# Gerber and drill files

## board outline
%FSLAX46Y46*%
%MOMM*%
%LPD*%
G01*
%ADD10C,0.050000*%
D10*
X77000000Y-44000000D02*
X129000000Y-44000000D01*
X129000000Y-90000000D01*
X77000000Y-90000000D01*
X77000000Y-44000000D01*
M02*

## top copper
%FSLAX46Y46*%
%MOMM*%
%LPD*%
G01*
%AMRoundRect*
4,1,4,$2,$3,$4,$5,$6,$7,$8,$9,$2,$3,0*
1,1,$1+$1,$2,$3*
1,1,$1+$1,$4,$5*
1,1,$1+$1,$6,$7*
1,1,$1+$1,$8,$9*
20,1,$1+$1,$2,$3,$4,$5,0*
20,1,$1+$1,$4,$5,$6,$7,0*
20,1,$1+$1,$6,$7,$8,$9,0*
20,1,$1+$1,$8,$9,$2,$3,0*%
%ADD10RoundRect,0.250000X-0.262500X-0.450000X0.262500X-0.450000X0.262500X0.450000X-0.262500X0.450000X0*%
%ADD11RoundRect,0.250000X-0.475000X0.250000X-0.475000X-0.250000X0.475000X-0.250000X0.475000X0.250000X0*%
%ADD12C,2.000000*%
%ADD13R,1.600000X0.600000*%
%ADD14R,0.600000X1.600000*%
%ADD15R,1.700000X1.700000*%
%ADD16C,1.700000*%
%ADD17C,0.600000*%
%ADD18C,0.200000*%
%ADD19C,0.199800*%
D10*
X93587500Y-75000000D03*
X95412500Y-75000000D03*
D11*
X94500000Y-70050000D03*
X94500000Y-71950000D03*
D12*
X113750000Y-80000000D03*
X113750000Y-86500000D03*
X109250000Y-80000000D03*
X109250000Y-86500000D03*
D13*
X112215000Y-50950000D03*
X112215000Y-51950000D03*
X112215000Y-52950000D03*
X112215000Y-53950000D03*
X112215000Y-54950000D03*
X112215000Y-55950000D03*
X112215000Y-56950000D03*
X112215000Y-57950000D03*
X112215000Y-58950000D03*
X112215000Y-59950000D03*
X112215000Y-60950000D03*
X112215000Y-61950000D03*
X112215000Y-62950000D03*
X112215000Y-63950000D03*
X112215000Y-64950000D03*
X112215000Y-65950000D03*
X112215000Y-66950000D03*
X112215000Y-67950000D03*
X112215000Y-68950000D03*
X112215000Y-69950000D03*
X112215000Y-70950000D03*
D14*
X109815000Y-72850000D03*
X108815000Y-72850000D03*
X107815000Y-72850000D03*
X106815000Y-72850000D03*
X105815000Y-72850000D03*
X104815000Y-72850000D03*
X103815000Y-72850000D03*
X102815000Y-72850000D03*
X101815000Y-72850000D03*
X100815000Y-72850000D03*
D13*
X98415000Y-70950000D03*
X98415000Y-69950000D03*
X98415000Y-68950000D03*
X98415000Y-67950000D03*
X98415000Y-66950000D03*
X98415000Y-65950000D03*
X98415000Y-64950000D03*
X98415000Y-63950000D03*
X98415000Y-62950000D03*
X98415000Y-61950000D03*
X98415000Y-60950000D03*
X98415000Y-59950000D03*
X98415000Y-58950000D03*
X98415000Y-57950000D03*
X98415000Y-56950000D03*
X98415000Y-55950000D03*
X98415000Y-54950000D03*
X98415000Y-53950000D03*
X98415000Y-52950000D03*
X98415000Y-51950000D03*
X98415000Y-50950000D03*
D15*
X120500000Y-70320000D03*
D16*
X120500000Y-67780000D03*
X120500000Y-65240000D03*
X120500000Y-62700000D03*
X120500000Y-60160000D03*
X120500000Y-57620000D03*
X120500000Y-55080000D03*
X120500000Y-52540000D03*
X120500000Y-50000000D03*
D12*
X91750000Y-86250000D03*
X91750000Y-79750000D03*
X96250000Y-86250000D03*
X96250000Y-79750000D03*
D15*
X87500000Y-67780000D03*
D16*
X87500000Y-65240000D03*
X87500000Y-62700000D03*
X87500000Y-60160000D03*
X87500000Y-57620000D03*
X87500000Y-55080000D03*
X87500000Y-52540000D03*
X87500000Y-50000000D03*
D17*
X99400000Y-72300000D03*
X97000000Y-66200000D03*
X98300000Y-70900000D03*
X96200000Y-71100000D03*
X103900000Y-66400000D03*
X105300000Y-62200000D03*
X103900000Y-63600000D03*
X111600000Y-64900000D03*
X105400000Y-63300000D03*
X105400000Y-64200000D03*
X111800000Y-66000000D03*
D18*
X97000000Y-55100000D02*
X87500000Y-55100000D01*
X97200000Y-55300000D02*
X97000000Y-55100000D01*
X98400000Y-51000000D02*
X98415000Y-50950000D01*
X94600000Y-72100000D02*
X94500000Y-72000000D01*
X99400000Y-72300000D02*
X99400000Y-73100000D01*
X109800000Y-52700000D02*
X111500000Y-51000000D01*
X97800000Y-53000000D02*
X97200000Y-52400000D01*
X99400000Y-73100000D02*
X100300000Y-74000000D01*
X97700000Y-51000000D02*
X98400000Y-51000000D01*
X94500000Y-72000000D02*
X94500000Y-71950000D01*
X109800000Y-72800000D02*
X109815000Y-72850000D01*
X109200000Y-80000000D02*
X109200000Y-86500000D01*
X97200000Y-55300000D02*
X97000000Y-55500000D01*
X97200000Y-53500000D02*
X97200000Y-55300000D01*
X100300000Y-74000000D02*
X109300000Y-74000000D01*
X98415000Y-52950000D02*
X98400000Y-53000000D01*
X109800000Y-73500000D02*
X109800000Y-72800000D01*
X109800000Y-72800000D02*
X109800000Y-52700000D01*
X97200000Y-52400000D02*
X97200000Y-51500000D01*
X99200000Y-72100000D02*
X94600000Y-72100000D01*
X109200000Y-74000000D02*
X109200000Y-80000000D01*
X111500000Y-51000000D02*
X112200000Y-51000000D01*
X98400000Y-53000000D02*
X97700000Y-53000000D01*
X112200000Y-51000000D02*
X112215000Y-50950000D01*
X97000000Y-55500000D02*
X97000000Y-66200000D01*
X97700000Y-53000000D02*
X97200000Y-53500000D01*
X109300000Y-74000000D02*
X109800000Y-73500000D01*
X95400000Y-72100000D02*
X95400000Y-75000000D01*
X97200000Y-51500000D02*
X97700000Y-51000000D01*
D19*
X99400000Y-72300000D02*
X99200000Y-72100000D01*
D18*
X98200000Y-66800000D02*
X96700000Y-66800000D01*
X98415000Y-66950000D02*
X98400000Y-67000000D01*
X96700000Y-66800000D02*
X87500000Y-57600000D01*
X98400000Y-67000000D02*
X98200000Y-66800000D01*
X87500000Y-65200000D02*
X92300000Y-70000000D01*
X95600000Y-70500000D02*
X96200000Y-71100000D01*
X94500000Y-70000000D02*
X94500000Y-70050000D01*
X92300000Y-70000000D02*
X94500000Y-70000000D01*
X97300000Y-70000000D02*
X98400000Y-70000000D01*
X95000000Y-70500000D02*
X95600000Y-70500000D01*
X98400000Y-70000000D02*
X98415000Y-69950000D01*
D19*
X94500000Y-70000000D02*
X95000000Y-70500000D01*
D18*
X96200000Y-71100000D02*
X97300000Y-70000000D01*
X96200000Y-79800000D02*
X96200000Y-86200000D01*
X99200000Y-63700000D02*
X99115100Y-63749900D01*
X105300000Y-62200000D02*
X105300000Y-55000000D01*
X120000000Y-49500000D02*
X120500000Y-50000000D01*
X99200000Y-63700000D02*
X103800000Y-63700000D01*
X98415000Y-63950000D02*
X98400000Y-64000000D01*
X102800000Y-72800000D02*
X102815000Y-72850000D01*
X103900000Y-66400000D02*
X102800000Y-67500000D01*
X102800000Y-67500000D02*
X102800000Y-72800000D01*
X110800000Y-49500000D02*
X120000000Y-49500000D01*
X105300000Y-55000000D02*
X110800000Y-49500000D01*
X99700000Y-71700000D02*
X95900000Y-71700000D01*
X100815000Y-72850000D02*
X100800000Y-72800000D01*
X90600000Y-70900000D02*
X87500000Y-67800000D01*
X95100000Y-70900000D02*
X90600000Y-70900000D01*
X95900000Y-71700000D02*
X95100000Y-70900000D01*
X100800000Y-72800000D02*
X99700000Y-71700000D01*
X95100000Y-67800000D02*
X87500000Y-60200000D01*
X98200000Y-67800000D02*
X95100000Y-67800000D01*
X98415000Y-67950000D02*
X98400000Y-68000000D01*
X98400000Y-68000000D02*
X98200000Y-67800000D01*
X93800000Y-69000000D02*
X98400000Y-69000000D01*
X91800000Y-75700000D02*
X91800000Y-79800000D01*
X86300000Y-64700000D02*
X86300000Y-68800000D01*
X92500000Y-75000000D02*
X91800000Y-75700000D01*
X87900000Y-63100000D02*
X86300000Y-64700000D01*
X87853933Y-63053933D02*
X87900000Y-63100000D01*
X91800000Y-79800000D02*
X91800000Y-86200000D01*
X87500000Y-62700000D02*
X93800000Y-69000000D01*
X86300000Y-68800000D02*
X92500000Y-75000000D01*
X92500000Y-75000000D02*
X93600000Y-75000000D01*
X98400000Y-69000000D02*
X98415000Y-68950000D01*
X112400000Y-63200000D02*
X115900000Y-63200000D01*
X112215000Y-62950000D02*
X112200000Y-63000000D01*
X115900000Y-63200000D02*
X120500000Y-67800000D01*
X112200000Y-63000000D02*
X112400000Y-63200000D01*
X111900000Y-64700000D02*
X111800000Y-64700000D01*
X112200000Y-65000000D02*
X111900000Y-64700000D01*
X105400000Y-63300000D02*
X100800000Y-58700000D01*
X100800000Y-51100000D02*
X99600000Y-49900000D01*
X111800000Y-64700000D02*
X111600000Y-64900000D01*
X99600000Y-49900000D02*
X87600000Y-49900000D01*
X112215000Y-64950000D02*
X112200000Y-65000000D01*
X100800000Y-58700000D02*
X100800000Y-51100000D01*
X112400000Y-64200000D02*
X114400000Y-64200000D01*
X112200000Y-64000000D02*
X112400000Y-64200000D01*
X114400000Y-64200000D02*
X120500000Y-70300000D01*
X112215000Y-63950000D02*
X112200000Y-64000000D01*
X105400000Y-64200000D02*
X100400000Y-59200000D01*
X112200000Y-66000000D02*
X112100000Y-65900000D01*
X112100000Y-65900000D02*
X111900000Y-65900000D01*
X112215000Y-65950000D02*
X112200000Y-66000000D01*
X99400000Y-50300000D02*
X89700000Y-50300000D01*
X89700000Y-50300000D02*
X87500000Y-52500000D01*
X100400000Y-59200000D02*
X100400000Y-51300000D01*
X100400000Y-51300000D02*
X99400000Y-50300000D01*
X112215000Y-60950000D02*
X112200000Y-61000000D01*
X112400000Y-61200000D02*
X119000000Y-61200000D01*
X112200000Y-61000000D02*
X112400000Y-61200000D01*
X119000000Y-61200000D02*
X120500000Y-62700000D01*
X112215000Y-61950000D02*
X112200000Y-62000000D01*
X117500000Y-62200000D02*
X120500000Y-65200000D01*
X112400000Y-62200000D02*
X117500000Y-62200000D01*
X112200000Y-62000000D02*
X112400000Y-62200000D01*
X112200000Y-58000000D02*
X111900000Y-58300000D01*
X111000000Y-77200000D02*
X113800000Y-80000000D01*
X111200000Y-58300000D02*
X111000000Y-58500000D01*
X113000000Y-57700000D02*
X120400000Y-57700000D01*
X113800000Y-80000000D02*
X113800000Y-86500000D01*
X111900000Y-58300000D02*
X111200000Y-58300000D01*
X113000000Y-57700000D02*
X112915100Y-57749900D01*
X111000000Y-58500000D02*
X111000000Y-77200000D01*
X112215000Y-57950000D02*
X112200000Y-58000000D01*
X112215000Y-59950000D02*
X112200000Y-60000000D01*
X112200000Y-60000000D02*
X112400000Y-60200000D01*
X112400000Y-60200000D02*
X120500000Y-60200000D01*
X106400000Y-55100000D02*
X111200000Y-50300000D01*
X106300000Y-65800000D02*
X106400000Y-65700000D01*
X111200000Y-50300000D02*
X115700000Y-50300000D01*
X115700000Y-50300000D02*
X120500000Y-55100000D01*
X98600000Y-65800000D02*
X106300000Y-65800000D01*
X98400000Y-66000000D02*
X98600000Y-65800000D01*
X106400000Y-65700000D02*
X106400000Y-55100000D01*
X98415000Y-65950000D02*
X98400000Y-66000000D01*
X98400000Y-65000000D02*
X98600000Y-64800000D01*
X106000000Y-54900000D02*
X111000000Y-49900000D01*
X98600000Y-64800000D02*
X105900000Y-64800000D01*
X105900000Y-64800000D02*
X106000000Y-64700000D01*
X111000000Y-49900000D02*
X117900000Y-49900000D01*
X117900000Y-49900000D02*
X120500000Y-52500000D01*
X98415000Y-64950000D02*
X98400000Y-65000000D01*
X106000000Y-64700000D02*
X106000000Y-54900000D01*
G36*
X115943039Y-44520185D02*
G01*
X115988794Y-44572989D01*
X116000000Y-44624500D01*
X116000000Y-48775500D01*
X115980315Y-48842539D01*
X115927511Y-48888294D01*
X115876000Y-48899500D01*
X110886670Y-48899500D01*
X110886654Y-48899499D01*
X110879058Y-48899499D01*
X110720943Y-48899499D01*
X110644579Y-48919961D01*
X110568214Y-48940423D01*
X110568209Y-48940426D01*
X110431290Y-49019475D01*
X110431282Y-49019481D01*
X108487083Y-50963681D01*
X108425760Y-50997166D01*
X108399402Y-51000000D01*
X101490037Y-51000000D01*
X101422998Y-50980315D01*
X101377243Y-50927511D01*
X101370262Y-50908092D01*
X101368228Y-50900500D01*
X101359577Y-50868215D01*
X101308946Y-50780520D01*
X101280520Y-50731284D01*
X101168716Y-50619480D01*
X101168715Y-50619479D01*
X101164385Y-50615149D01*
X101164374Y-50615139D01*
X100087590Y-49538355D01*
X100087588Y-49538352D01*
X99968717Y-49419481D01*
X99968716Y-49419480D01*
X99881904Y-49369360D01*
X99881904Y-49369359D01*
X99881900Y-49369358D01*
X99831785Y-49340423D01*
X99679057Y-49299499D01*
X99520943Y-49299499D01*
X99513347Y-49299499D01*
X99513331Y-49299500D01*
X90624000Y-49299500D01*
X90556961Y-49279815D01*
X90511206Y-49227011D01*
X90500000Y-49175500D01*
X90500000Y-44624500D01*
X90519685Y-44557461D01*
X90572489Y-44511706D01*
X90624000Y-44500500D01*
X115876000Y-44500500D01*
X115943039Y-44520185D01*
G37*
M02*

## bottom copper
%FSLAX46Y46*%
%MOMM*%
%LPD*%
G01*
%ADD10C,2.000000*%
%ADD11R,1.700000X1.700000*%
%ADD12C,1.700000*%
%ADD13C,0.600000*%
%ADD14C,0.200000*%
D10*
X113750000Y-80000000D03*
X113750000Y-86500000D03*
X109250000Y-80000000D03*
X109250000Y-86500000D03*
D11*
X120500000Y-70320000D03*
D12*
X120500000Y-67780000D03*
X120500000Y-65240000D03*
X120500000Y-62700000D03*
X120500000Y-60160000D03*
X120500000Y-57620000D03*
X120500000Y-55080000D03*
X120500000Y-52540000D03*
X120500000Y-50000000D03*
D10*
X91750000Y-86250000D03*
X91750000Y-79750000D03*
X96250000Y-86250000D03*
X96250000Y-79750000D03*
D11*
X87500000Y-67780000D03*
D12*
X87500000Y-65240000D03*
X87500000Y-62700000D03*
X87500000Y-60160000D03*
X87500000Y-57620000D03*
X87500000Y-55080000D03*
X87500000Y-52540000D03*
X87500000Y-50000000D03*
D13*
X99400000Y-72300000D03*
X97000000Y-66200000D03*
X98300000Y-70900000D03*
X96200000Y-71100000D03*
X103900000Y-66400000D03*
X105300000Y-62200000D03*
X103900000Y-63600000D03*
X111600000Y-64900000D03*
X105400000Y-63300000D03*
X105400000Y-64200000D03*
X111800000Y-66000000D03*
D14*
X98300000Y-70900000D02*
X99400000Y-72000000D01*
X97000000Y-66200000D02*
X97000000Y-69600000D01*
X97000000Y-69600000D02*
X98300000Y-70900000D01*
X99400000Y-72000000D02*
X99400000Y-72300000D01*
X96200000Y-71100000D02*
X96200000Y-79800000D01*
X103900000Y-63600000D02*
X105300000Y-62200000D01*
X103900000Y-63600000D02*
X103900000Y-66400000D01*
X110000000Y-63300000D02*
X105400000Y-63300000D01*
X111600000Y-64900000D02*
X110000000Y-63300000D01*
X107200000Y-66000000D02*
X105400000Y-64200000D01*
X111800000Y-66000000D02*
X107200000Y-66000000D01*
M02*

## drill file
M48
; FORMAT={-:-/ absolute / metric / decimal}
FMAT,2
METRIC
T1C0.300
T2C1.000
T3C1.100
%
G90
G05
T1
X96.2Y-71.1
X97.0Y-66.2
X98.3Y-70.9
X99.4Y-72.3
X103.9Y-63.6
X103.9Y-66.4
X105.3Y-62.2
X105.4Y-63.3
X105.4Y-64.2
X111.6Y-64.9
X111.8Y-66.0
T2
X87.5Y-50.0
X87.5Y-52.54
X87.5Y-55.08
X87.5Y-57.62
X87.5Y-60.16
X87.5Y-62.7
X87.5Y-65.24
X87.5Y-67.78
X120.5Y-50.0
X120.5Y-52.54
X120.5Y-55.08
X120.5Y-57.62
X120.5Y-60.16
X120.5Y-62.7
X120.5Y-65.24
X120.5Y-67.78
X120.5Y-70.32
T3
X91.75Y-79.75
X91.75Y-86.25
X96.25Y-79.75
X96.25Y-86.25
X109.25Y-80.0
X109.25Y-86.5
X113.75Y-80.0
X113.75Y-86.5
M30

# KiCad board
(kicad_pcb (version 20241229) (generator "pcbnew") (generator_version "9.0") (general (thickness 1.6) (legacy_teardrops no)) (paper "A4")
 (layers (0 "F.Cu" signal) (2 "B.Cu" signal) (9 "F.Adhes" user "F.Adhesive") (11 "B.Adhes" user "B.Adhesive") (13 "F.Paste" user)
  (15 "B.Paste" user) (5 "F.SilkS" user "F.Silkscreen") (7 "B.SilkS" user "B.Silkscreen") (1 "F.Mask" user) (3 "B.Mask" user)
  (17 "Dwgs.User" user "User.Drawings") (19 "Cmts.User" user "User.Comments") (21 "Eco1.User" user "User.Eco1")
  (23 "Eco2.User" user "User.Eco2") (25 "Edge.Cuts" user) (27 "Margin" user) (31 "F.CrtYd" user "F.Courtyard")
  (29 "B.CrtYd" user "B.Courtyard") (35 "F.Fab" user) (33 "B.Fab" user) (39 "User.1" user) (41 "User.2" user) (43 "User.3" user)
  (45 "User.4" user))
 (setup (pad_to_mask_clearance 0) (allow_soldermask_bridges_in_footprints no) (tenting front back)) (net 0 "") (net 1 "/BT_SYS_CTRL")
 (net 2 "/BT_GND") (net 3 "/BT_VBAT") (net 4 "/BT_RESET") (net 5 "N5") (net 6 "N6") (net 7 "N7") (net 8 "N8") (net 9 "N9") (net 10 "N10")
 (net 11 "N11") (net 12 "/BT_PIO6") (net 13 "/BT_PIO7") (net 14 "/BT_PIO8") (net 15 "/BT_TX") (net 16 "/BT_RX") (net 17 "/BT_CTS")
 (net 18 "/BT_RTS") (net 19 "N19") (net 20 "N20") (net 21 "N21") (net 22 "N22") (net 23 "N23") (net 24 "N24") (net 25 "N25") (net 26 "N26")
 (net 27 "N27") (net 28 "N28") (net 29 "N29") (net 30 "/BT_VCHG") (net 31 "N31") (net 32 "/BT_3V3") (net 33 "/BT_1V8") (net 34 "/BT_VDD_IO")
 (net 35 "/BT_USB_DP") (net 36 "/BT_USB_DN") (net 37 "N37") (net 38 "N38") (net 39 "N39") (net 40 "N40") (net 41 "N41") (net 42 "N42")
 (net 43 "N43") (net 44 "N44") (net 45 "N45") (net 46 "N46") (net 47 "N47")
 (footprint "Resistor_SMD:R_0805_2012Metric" (layer "F.Cu") (at 94.5 75)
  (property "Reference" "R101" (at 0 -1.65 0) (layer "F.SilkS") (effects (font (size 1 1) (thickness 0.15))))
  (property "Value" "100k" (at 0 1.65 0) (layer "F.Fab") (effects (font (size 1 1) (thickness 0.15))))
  (pad "1" smd roundrect (at -0.9125 0) (size 1.025 1.4) (layers "F.Cu" "F.Mask" "F.Paste") (roundrect_rratio 0.243902)
   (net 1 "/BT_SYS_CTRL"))
  (pad "2" smd roundrect (at 0.9125 0) (size 1.025 1.4) (layers "F.Cu" "F.Mask" "F.Paste") (roundrect_rratio 0.243902) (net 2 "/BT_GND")))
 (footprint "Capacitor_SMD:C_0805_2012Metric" (layer "F.Cu") (at 94.5 71 -90)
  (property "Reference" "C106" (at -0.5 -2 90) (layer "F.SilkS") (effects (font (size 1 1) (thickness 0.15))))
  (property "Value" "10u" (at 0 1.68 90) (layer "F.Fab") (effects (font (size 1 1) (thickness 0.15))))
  (pad "1" smd roundrect (at -0.95 0 270) (size 1 1.45) (layers "F.Cu" "F.Mask" "F.Paste") (roundrect_rratio 0.25) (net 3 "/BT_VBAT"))
  (pad "2" smd roundrect (at 0.95 0 270) (size 1 1.45) (layers "F.Cu" "F.Mask" "F.Paste") (roundrect_rratio 0.25) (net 2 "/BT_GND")))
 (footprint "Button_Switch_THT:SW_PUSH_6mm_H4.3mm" (layer "F.Cu") (at 113.75 80 -90)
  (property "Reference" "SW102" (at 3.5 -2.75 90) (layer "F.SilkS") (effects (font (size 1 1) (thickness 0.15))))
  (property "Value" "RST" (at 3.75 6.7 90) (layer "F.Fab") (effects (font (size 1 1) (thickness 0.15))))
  (pad "1" thru_hole circle (at 0 0) (size 2 2) (drill 1.1) (layers "*.Cu" "*.Mask") (remove_unused_layers no) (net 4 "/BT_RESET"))
  (pad "1" thru_hole circle (at 6.5 0) (size 2 2) (drill 1.1) (layers "*.Cu" "*.Mask") (remove_unused_layers no) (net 4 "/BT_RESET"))
  (pad "2" thru_hole circle (at 0 4.5) (size 2 2) (drill 1.1) (layers "*.Cu" "*.Mask") (remove_unused_layers no) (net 2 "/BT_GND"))
  (pad "2" thru_hole circle (at 6.5 4.5) (size 2 2) (drill 1.1) (layers "*.Cu" "*.Mask") (remove_unused_layers no) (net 2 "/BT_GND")))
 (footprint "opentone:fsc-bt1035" (layer "F.Cu") (at 105.315 59 180)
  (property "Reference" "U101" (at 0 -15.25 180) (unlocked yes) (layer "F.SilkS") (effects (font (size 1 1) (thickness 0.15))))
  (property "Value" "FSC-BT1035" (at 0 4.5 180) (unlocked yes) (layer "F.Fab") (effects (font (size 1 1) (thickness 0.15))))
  (pad "1" smd rect (at -6.9 8.05 180) (size 1.6 0.6) (layers "F.Cu" "F.Mask" "F.Paste") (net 2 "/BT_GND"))
  (pad "2" smd rect (at -6.9 7.05 180) (size 1.6 0.6) (layers "F.Cu" "F.Mask" "F.Paste") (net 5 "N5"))
  (pad "3" smd rect (at -6.9 6.05 180) (size 1.6 0.6) (layers "F.Cu" "F.Mask" "F.Paste") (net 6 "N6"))
  (pad "4" smd rect (at -6.9 5.05 180) (size 1.6 0.6) (layers "F.Cu" "F.Mask" "F.Paste") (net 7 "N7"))
  (pad "5" smd rect (at -6.9 4.05 180) (size 1.6 0.6) (layers "F.Cu" "F.Mask" "F.Paste") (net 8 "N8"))
  (pad "6" smd rect (at -6.9 3.05 180) (size 1.6 0.6) (layers "F.Cu" "F.Mask" "F.Paste") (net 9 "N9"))
  (pad "7" smd rect (at -6.9 2.05 180) (size 1.6 0.6) (layers "F.Cu" "F.Mask" "F.Paste") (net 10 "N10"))
  (pad "8" smd rect (at -6.9 1.05 180) (size 1.6 0.6) (layers "F.Cu" "F.Mask" "F.Paste") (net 4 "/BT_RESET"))
  (pad "9" smd rect (at -6.9 0.05 180) (size 1.6 0.6) (layers "F.Cu" "F.Mask" "F.Paste") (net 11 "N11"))
  (pad "10" smd rect (at -6.9 -0.95 180) (size 1.6 0.6) (layers "F.Cu" "F.Mask" "F.Paste") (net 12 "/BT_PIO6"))
  (pad "11" smd rect (at -6.9 -1.95 180) (size 1.6 0.6) (layers "F.Cu" "F.Mask" "F.Paste") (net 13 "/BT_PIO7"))
  (pad "12" smd rect (at -6.9 -2.95 180) (size 1.6 0.6) (layers "F.Cu" "F.Mask" "F.Paste") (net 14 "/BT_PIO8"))
  (pad "13" smd rect (at -6.9 -3.95 180) (size 1.6 0.6) (layers "F.Cu" "F.Mask" "F.Paste") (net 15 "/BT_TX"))
  (pad "14" smd rect (at -6.9 -4.95 180) (size 1.6 0.6) (layers "F.Cu" "F.Mask" "F.Paste") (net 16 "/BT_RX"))
  (pad "15" smd rect (at -6.9 -5.95 180) (size 1.6 0.6) (layers "F.Cu" "F.Mask" "F.Paste") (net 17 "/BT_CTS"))
  (pad "16" smd rect (at -6.9 -6.95 180) (size 1.6 0.6) (layers "F.Cu" "F.Mask" "F.Paste") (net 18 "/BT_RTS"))
  (pad "17" smd rect (at -6.9 -7.95 180) (size 1.6 0.6) (layers "F.Cu" "F.Mask" "F.Paste") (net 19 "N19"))
  (pad "18" smd rect (at -6.9 -8.95 180) (size 1.6 0.6) (layers "F.Cu" "F.Mask" "F.Paste") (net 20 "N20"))
  (pad "19" smd rect (at -6.9 -9.95 180) (size 1.6 0.6) (layers "F.Cu" "F.Mask" "F.Paste") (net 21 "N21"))
  (pad "20" smd rect (at -6.9 -10.95 180) (size 1.6 0.6) (layers "F.Cu" "F.Mask" "F.Paste") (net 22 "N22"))
  (pad "21" smd rect (at -6.9 -11.95 180) (size 1.6 0.6) (layers "F.Cu" "F.Mask" "F.Paste") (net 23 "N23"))
  (pad "22" smd rect (at -4.5 -13.85 180) (size 0.6 1.6) (layers "F.Cu" "F.Mask" "F.Paste") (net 2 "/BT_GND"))
  (pad "23" smd rect (at -3.5 -13.85 180) (size 0.6 1.6) (layers "F.Cu" "F.Mask" "F.Paste") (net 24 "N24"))
  (pad "24" smd rect (at -2.5 -13.85 180) (size 0.6 1.6) (layers "F.Cu" "F.Mask" "F.Paste") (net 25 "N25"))
  (pad "25" smd rect (at -1.5 -13.85 180) (size 0.6 1.6) (layers "F.Cu" "F.Mask" "F.Paste") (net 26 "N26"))
  (pad "26" smd rect (at -0.5 -13.85 180) (size 0.6 1.6) (layers "F.Cu" "F.Mask" "F.Paste") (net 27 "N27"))
  (pad "27" smd rect (at 0.5 -13.85 180) (size 0.6 1.6) (layers "F.Cu" "F.Mask" "F.Paste") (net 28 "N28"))
  (pad "28" smd rect (at 1.5 -13.85 180) (size 0.6 1.6) (layers "F.Cu" "F.Mask" "F.Paste") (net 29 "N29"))
  (pad "29" smd rect (at 2.5 -13.85 180) (size 0.6 1.6) (layers "F.Cu" "F.Mask" "F.Paste") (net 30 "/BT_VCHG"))
  (pad "30" smd rect (at 3.5 -13.85 180) (size 0.6 1.6) (layers "F.Cu" "F.Mask" "F.Paste") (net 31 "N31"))
  (pad "31" smd rect (at 4.5 -13.85 180) (size 0.6 1.6) (layers "F.Cu" "F.Mask" "F.Paste") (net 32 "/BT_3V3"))
  (pad "32" smd rect (at 6.9 -11.95 180) (size 1.6 0.6) (layers "F.Cu" "F.Mask" "F.Paste") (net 2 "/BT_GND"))
  (pad "33" smd rect (at 6.9 -10.95 180) (size 1.6 0.6) (layers "F.Cu" "F.Mask" "F.Paste") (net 3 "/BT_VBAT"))
  (pad "34" smd rect (at 6.9 -9.95 180) (size 1.6 0.6) (layers "F.Cu" "F.Mask" "F.Paste") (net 1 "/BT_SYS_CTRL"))
  (pad "35" smd rect (at 6.9 -8.95 180) (size 1.6 0.6) (layers "F.Cu" "F.Mask" "F.Paste") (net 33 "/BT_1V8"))
  (pad "36" smd rect (at 6.9 -7.95 180) (size 1.6 0.6) (layers "F.Cu" "F.Mask" "F.Paste") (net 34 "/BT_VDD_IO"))
  (pad "37" smd rect (at 6.9 -6.95 180) (size 1.6 0.6) (layers "F.Cu" "F.Mask" "F.Paste") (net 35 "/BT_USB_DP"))
  (pad "38" smd rect (at 6.9 -5.95 180) (size 1.6 0.6) (layers "F.Cu" "F.Mask" "F.Paste") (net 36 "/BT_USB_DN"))
  (pad "39" smd rect (at 6.9 -4.95 180) (size 1.6 0.6) (layers "F.Cu" "F.Mask" "F.Paste") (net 30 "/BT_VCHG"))
  (pad "40" smd rect (at 6.9 -3.95 180) (size 1.6 0.6) (layers "F.Cu" "F.Mask" "F.Paste") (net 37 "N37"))
  (pad "41" smd rect (at 6.9 -2.95 180) (size 1.6 0.6) (layers "F.Cu" "F.Mask" "F.Paste") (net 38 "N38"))
  (pad "42" smd rect (at 6.9 -1.95 180) (size 1.6 0.6) (layers "F.Cu" "F.Mask" "F.Paste") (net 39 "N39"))
  (pad "43" smd rect (at 6.9 -0.95 180) (size 1.6 0.6) (layers "F.Cu" "F.Mask" "F.Paste") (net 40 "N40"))
  (pad "44" smd rect (at 6.9 0.05 180) (size 1.6 0.6) (layers "F.Cu" "F.Mask" "F.Paste") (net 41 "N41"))
  (pad "45" smd rect (at 6.9 1.05 180) (size 1.6 0.6) (layers "F.Cu" "F.Mask" "F.Paste") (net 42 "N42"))
  (pad "46" smd rect (at 6.9 2.05 180) (size 1.6 0.6) (layers "F.Cu" "F.Mask" "F.Paste") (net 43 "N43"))
  (pad "47" smd rect (at 6.9 3.05 180) (size 1.6 0.6) (layers "F.Cu" "F.Mask" "F.Paste") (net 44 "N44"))
  (pad "48" smd rect (at 6.9 4.05 180) (size 1.6 0.6) (layers "F.Cu" "F.Mask" "F.Paste") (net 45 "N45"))
  (pad "49" smd rect (at 6.9 5.05 180) (size 1.6 0.6) (layers "F.Cu" "F.Mask" "F.Paste") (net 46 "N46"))
  (pad "50" smd rect (at 6.9 6.05 180) (size 1.6 0.6) (layers "F.Cu" "F.Mask" "F.Paste") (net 2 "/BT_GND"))
  (pad "51" smd rect (at 6.9 7.05 180) (size 1.6 0.6) (layers "F.Cu" "F.Mask" "F.Paste") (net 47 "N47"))
  (pad "52" smd rect (at 6.9 8.05 180) (size 1.6 0.6) (layers "F.Cu" "F.Mask" "F.Paste") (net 2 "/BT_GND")))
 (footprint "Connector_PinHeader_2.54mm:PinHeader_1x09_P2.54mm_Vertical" (layer "F.Cu") (at 120.5 70.32 180)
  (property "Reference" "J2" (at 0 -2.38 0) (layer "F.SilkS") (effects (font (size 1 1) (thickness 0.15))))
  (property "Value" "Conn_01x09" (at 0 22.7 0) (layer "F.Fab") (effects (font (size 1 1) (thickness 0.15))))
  (pad "1" thru_hole rect (at 0 0 180) (size 1.7 1.7) (drill 1) (layers "*.Cu" "*.Mask") (remove_unused_layers no) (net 16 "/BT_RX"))
  (pad "2" thru_hole circle (at 0 2.54 180) (size 1.7 1.7) (drill 1) (layers "*.Cu" "*.Mask") (remove_unused_layers no) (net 15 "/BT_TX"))
  (pad "3" thru_hole circle (at 0 5.08 180) (size 1.7 1.7) (drill 1) (layers "*.Cu" "*.Mask") (remove_unused_layers no) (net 14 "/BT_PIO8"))
  (pad "4" thru_hole circle (at 0 7.62 180) (size 1.7 1.7) (drill 1) (layers "*.Cu" "*.Mask") (remove_unused_layers no) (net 13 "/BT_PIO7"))
  (pad "5" thru_hole circle (at 0 10.16 180) (size 1.7 1.7) (drill 1) (layers "*.Cu" "*.Mask") (remove_unused_layers no) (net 12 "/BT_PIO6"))
  (pad "6" thru_hole circle (at 0 12.7 180) (size 1.7 1.7) (drill 1) (layers "*.Cu" "*.Mask") (remove_unused_layers no) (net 4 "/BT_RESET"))
  (pad "7" thru_hole circle (at 0 15.24 180) (size 1.7 1.7) (drill 1) (layers "*.Cu" "*.Mask") (remove_unused_layers no)
   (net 35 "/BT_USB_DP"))
  (pad "8" thru_hole circle (at 0 17.78 180) (size 1.7 1.7) (drill 1) (layers "*.Cu" "*.Mask") (remove_unused_layers no)
   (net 36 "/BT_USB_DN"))
  (pad "9" thru_hole circle (at 0 20.32 180) (size 1.7 1.7) (drill 1) (layers "*.Cu" "*.Mask") (remove_unused_layers no) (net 30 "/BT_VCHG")))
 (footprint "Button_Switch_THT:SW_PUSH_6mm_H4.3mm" (layer "F.Cu") (at 91.75 86.25 90)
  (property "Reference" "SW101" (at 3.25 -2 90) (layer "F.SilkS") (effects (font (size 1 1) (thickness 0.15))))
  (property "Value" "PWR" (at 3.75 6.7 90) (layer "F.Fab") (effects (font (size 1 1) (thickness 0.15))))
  (pad "1" thru_hole circle (at 0 0 180) (size 2 2) (drill 1.1) (layers "*.Cu" "*.Mask") (remove_unused_layers no) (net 1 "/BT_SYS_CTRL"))
  (pad "1" thru_hole circle (at 6.5 0 180) (size 2 2) (drill 1.1) (layers "*.Cu" "*.Mask") (remove_unused_layers no) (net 1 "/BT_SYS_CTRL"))
  (pad "2" thru_hole circle (at 0 4.5 180) (size 2 2) (drill 1.1) (layers "*.Cu" "*.Mask") (remove_unused_layers no) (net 3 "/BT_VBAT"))
  (pad "2" thru_hole circle (at 6.5 4.5 180) (size 2 2) (drill 1.1) (layers "*.Cu" "*.Mask") (remove_unused_layers no) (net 3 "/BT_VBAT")))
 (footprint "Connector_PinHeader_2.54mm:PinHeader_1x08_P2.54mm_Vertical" (layer "F.Cu") (at 87.5 67.78 180)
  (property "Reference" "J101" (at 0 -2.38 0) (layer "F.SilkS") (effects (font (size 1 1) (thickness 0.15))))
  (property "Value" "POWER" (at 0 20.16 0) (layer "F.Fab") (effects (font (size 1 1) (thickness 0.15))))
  (pad "1" thru_hole rect (at 0 0 180) (size 1.7 1.7) (drill 1) (layers "*.Cu" "*.Mask") (remove_unused_layers no) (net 32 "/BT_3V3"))
  (pad "2" thru_hole circle (at 0 2.54 180) (size 1.7 1.7) (drill 1) (layers "*.Cu" "*.Mask") (remove_unused_layers no) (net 3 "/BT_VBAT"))
  (pad "3" thru_hole circle (at 0 5.08 180) (size 1.7 1.7) (drill 1) (layers "*.Cu" "*.Mask") (remove_unused_layers no)
   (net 1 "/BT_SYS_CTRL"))
  (pad "4" thru_hole circle (at 0 7.62 180) (size 1.7 1.7) (drill 1) (layers "*.Cu" "*.Mask") (remove_unused_layers no) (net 33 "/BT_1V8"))
  (pad "5" thru_hole circle (at 0 10.16 180) (size 1.7 1.7) (drill 1) (layers "*.Cu" "*.Mask") (remove_unused_layers no)
   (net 34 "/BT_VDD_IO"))
  (pad "6" thru_hole circle (at 0 12.7 180) (size 1.7 1.7) (drill 1) (layers "*.Cu" "*.Mask") (remove_unused_layers no) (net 2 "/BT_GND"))
  (pad "7" thru_hole circle (at 0 15.24 180) (size 1.7 1.7) (drill 1) (layers "*.Cu" "*.Mask") (remove_unused_layers no) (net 18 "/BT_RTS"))
  (pad "8" thru_hole circle (at 0 17.78 180) (size 1.7 1.7) (drill 1) (layers "*.Cu" "*.Mask") (remove_unused_layers no) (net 17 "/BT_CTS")))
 (gr_rect (start 77 44) (end 129 90) (stroke (width 0.05) (type default)) (fill no) (layer "Edge.Cuts"))
 (segment (start 97 55.1) (end 87.5 55.1) (width 0.2) (layer "F.Cu") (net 2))
 (segment (start 97.2 55.3) (end 97 55.1) (width 0.2) (layer "F.Cu") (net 2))
 (segment (start 98.4 51) (end 98.415 50.95) (width 0.2) (layer "F.Cu") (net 2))
 (segment (start 94.6 72.1) (end 94.5 72) (width 0.2) (layer "F.Cu") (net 2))
 (segment (start 99.4 72.3) (end 99.4 73.1) (width 0.2) (layer "F.Cu") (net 2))
 (segment (start 109.8 52.7) (end 111.5 51) (width 0.2) (layer "F.Cu") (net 2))
 (segment (start 97.8 53) (end 97.2 52.4) (width 0.2) (layer "F.Cu") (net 2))
 (segment (start 99.4 73.1) (end 100.3 74) (width 0.2) (layer "F.Cu") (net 2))
 (segment (start 97.7 51) (end 98.4 51) (width 0.2) (layer "F.Cu") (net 2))
 (segment (start 94.5 72) (end 94.5 71.95) (width 0.2) (layer "F.Cu") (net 2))
 (segment (start 109.8 72.8) (end 109.815 72.85) (width 0.2) (layer "F.Cu") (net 2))
 (segment (start 109.2 80) (end 109.2 86.5) (width 0.2) (layer "F.Cu") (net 2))
 (segment (start 97.2 55.3) (end 97 55.5) (width 0.2) (layer "F.Cu") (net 2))
 (segment (start 97.2 53.5) (end 97.2 55.3) (width 0.2) (layer "F.Cu") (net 2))
 (segment (start 100.3 74) (end 109.3 74) (width 0.2) (layer "F.Cu") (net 2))
 (segment (start 98.415 52.95) (end 98.4 53) (width 0.2) (layer "F.Cu") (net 2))
 (segment (start 109.8 73.5) (end 109.8 72.8) (width 0.2) (layer "F.Cu") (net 2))
 (segment (start 109.8 72.8) (end 109.8 52.7) (width 0.2) (layer "F.Cu") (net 2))
 (segment (start 97.2 52.4) (end 97.2 51.5) (width 0.2) (layer "F.Cu") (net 2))
 (segment (start 99.2 72.1) (end 94.6 72.1) (width 0.2) (layer "F.Cu") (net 2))
 (segment (start 109.2 74) (end 109.2 80) (width 0.2) (layer "F.Cu") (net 2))
 (segment (start 111.5 51) (end 112.2 51) (width 0.2) (layer "F.Cu") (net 2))
 (segment (start 98.4 53) (end 97.7 53) (width 0.2) (layer "F.Cu") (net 2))
 (segment (start 112.2 51) (end 112.215 50.95) (width 0.2) (layer "F.Cu") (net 2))
 (segment (start 97 55.5) (end 97 66.2) (width 0.2) (layer "F.Cu") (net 2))
 (segment (start 97.7 53) (end 97.2 53.5) (width 0.2) (layer "F.Cu") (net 2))
 (segment (start 109.3 74) (end 109.8 73.5) (width 0.2) (layer "F.Cu") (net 2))
 (segment (start 95.4 72.1) (end 95.4 75) (width 0.2) (layer "F.Cu") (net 2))
 (segment (start 97.2 51.5) (end 97.7 51) (width 0.2) (layer "F.Cu") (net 2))
 (segment (start 99.4 72.3) (end 99.2 72.1) (width 0.1998) (layer "F.Cu") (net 2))
 (via (at 99.4 72.3) (size 0.6) (drill 0.3) (layers "F.Cu" "B.Cu") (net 2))
 (via (at 97 66.2) (size 0.6) (drill 0.3) (layers "F.Cu" "B.Cu") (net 2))
 (via (at 98.3 70.9) (size 0.6) (drill 0.3) (layers "F.Cu" "B.Cu") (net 2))
 (segment (start 98.3 70.9) (end 99.4 72) (width 0.2) (layer "B.Cu") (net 2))
 (segment (start 97 66.2) (end 97 69.6) (width 0.2) (layer "B.Cu") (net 2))
 (segment (start 97 69.6) (end 98.3 70.9) (width 0.2) (layer "B.Cu") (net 2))
 (segment (start 99.4 72) (end 99.4 72.3) (width 0.2) (layer "B.Cu") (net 2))
 (segment (start 98.2 66.8) (end 96.7 66.8) (width 0.2) (layer "F.Cu") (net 34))
 (segment (start 98.415 66.95) (end 98.4 67) (width 0.2) (layer "F.Cu") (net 34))
 (segment (start 96.7 66.8) (end 87.5 57.6) (width 0.2) (layer "F.Cu") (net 34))
 (segment (start 98.4 67) (end 98.2 66.8) (width 0.2) (layer "F.Cu") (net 34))
 (segment (start 87.5 65.2) (end 92.3 70) (width 0.2) (layer "F.Cu") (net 3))
 (segment (start 95.6 70.5) (end 96.2 71.1) (width 0.2) (layer "F.Cu") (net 3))
 (segment (start 94.5 70) (end 94.5 70.05) (width 0.2) (layer "F.Cu") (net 3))
 (segment (start 92.3 70) (end 94.5 70) (width 0.2) (layer "F.Cu") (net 3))
 (segment (start 97.3 70) (end 98.4 70) (width 0.2) (layer "F.Cu") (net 3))
 (segment (start 95 70.5) (end 95.6 70.5) (width 0.2) (layer "F.Cu") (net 3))
 (segment (start 98.4 70) (end 98.415 69.95) (width 0.2) (layer "F.Cu") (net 3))
 (segment (start 94.5 70) (end 95 70.5) (width 0.1998) (layer "F.Cu") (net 3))
 (segment (start 96.2 71.1) (end 97.3 70) (width 0.2) (layer "F.Cu") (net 3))
 (segment (start 96.2 79.8) (end 96.2 86.2) (width 0.2) (layer "F.Cu") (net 3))
 (via (at 96.2 71.1) (size 0.6) (drill 0.3) (layers "F.Cu" "B.Cu") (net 3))
 (segment (start 96.2 71.1) (end 96.2 79.8) (width 0.2) (layer "B.Cu") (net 3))
 (segment (start 99.2 63.7) (end 99.1151 63.7499) (width 0.2) (layer "F.Cu") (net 30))
 (segment (start 105.3 62.2) (end 105.3 55) (width 0.2) (layer "F.Cu") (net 30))
 (segment (start 120 49.5) (end 120.5 50) (width 0.2) (layer "F.Cu") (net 30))
 (segment (start 99.2 63.7) (end 103.8 63.7) (width 0.2) (layer "F.Cu") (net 30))
 (segment (start 98.415 63.95) (end 98.4 64) (width 0.2) (layer "F.Cu") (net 30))
 (segment (start 102.8 72.8) (end 102.815 72.85) (width 0.2) (layer "F.Cu") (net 30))
 (segment (start 103.9 66.4) (end 102.8 67.5) (width 0.2) (layer "F.Cu") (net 30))
 (segment (start 102.8 67.5) (end 102.8 72.8) (width 0.2) (layer "F.Cu") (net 30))
 (segment (start 110.8 49.5) (end 120 49.5) (width 0.2) (layer "F.Cu") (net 30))
 (segment (start 105.3 55) (end 110.8 49.5) (width 0.2) (layer "F.Cu") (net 30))
 (via (at 103.9 66.4) (size 0.6) (drill 0.3) (layers "F.Cu" "B.Cu") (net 30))
 (via (at 105.3 62.2) (size 0.6) (drill 0.3) (layers "F.Cu" "B.Cu") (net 30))
 (via (at 103.9 63.6) (size 0.6) (drill 0.3) (layers "F.Cu" "B.Cu") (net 30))
 (segment (start 103.9 63.6) (end 105.3 62.2) (width 0.2) (layer "B.Cu") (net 30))
 (segment (start 103.9 63.6) (end 103.9 66.4) (width 0.2) (layer "B.Cu") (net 30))
 (segment (start 99.7 71.7) (end 95.9 71.7) (width 0.2) (layer "F.Cu") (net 32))
 (segment (start 100.815 72.85) (end 100.8 72.8) (width 0.2) (layer "F.Cu") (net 32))
 (segment (start 90.6 70.9) (end 87.5 67.8) (width 0.2) (layer "F.Cu") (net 32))
 (segment (start 95.1 70.9) (end 90.6 70.9) (width 0.2) (layer "F.Cu") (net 32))
 (segment (start 95.9 71.7) (end 95.1 70.9) (width 0.2) (layer "F.Cu") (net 32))
 (segment (start 100.8 72.8) (end 99.7 71.7) (width 0.2) (layer "F.Cu") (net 32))
 (segment (start 95.1 67.8) (end 87.5 60.2) (width 0.2) (layer "F.Cu") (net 33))
 (segment (start 98.2 67.8) (end 95.1 67.8) (width 0.2) (layer "F.Cu") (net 33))
 (segment (start 98.415 67.95) (end 98.4 68) (width 0.2) (layer "F.Cu") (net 33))
 (segment (start 98.4 68) (end 98.2 67.8) (width 0.2) (layer "F.Cu") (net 33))
 (segment (start 93.8 69) (end 98.4 69) (width 0.2) (layer "F.Cu") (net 1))
 (segment (start 91.8 75.7) (end 91.8 79.8) (width 0.2) (layer "F.Cu") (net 1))
 (segment (start 86.3 64.7) (end 86.3 68.8) (width 0.2) (layer "F.Cu") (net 1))
 (segment (start 92.5 75) (end 91.8 75.7) (width 0.2) (layer "F.Cu") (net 1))
 (segment (start 87.9 63.1) (end 86.3 64.7) (width 0.2) (layer "F.Cu") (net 1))
 (segment (start 87.853933 63.053933) (end 87.9 63.1) (width 0.2) (layer "F.Cu") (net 1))
 (segment (start 91.8 79.8) (end 91.8 86.2) (width 0.2) (layer "F.Cu") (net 1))
 (segment (start 87.5 62.7) (end 93.8 69) (width 0.2) (layer "F.Cu") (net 1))
 (segment (start 86.3 68.8) (end 92.5 75) (width 0.2) (layer "F.Cu") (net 1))
 (segment (start 92.5 75) (end 93.6 75) (width 0.2) (layer "F.Cu") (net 1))
 (segment (start 98.4 69) (end 98.415 68.95) (width 0.2) (layer "F.Cu") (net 1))
 (segment (start 112.4 63.2) (end 115.9 63.2) (width 0.2) (layer "F.Cu") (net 15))
 (segment (start 112.215 62.95) (end 112.2 63) (width 0.2) (layer "F.Cu") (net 15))
 (segment (start 115.9 63.2) (end 120.5 67.8) (width 0.2) (layer "F.Cu") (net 15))
 (segment (start 112.2 63) (end 112.4 63.2) (width 0.2) (layer "F.Cu") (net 15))
 (segment (start 111.9 64.7) (end 111.8 64.7) (width 0.2) (layer "F.Cu") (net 17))
 (segment (start 112.2 65) (end 111.9 64.7) (width 0.2) (layer "F.Cu") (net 17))
 (segment (start 105.4 63.3) (end 100.8 58.7) (width 0.2) (layer "F.Cu") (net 17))
 (segment (start 100.8 51.1) (end 99.6 49.9) (width 0.2) (layer "F.Cu") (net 17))
 (segment (start 111.8 64.7) (end 111.6 64.9) (width 0.2) (layer "F.Cu") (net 17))
 (segment (start 99.6 49.9) (end 87.6 49.9) (width 0.2) (layer "F.Cu") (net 17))
 (segment (start 112.215 64.95) (end 112.2 65) (width 0.2) (layer "F.Cu") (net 17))
 (segment (start 100.8 58.7) (end 100.8 51.1) (width 0.2) (layer "F.Cu") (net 17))
 (via (at 111.6 64.9) (size 0.6) (drill 0.3) (layers "F.Cu" "B.Cu") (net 17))
 (via (at 105.4 63.3) (size 0.6) (drill 0.3) (layers "F.Cu" "B.Cu") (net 17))
 (segment (start 110 63.3) (end 105.4 63.3) (width 0.2) (layer "B.Cu") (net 17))
 (segment (start 111.6 64.9) (end 110 63.3) (width 0.2) (layer "B.Cu") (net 17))
 (segment (start 112.4 64.2) (end 114.4 64.2) (width 0.2) (layer "F.Cu") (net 16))
 (segment (start 112.2 64) (end 112.4 64.2) (width 0.2) (layer "F.Cu") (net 16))
 (segment (start 114.4 64.2) (end 120.5 70.3) (width 0.2) (layer "F.Cu") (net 16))
 (segment (start 112.215 63.95) (end 112.2 64) (width 0.2) (layer "F.Cu") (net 16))
 (segment (start 105.4 64.2) (end 100.4 59.2) (width 0.2) (layer "F.Cu") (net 18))
 (segment (start 112.2 66) (end 112.1 65.9) (width 0.2) (layer "F.Cu") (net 18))
 (segment (start 112.1 65.9) (end 111.9 65.9) (width 0.2) (layer "F.Cu") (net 18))
 (segment (start 112.215 65.95) (end 112.2 66) (width 0.2) (layer "F.Cu") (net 18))
 (segment (start 99.4 50.3) (end 89.7 50.3) (width 0.2) (layer "F.Cu") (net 18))
 (segment (start 89.7 50.3) (end 87.5 52.5) (width 0.2) (layer "F.Cu") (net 18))
 (segment (start 100.4 59.2) (end 100.4 51.3) (width 0.2) (layer "F.Cu") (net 18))
 (segment (start 100.4 51.3) (end 99.4 50.3) (width 0.2) (layer "F.Cu") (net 18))
 (via (at 105.4 64.2) (size 0.6) (drill 0.3) (layers "F.Cu" "B.Cu") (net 18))
 (via (at 111.8 66) (size 0.6) (drill 0.3) (layers "F.Cu" "B.Cu") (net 18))
 (segment (start 107.2 66) (end 105.4 64.2) (width 0.2) (layer "B.Cu") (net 18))
 (segment (start 111.8 66) (end 107.2 66) (width 0.2) (layer "B.Cu") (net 18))
 (segment (start 112.215 60.95) (end 112.2 61) (width 0.2) (layer "F.Cu") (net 13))
 (segment (start 112.4 61.2) (end 119 61.2) (width 0.2) (layer "F.Cu") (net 13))
 (segment (start 112.2 61) (end 112.4 61.2) (width 0.2) (layer "F.Cu") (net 13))
 (segment (start 119 61.2) (end 120.5 62.7) (width 0.2) (layer "F.Cu") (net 13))
 (segment (start 112.215 61.95) (end 112.2 62) (width 0.2) (layer "F.Cu") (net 14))
 (segment (start 117.5 62.2) (end 120.5 65.2) (width 0.2) (layer "F.Cu") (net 14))
 (segment (start 112.4 62.2) (end 117.5 62.2) (width 0.2) (layer "F.Cu") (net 14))
 (segment (start 112.2 62) (end 112.4 62.2) (width 0.2) (layer "F.Cu") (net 14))
 (segment (start 112.2 58) (end 111.9 58.3) (width 0.2) (layer "F.Cu") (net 4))
 (segment (start 111 77.2) (end 113.8 80) (width 0.2) (layer "F.Cu") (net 4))
 (segment (start 111.2 58.3) (end 111 58.5) (width 0.2) (layer "F.Cu") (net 4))
 (segment (start 113 57.7) (end 120.4 57.7) (width 0.2) (layer "F.Cu") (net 4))
 (segment (start 113.8 80) (end 113.8 86.5) (width 0.2) (layer "F.Cu") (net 4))
 (segment (start 111.9 58.3) (end 111.2 58.3) (width 0.2) (layer "F.Cu") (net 4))
 (segment (start 113 57.7) (end 112.9151 57.7499) (width 0.2) (layer "F.Cu") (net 4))
 (segment (start 111 58.5) (end 111 77.2) (width 0.2) (layer "F.Cu") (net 4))
 (segment (start 112.215 57.95) (end 112.2 58) (width 0.2) (layer "F.Cu") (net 4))
 (segment (start 112.215 59.95) (end 112.2 60) (width 0.2) (layer "F.Cu") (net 12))
 (segment (start 112.2 60) (end 112.4 60.2) (width 0.2) (layer "F.Cu") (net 12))
 (segment (start 112.4 60.2) (end 120.5 60.2) (width 0.2) (layer "F.Cu") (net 12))
 (segment (start 106.4 55.1) (end 111.2 50.3) (width 0.2) (layer "F.Cu") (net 35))
 (segment (start 106.3 65.8) (end 106.4 65.7) (width 0.2) (layer "F.Cu") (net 35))
 (segment (start 111.2 50.3) (end 115.7 50.3) (width 0.2) (layer "F.Cu") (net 35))
 (segment (start 115.7 50.3) (end 120.5 55.1) (width 0.2) (layer "F.Cu") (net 35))
 (segment (start 98.6 65.8) (end 106.3 65.8) (width 0.2) (layer "F.Cu") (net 35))
 (segment (start 98.4 66) (end 98.6 65.8) (width 0.2) (layer "F.Cu") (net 35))
 (segment (start 106.4 65.7) (end 106.4 55.1) (width 0.2) (layer "F.Cu") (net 35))
 (segment (start 98.415 65.95) (end 98.4 66) (width 0.2) (layer "F.Cu") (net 35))
 (segment (start 98.4 65) (end 98.6 64.8) (width 0.2) (layer "F.Cu") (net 36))
 (segment (start 106 54.9) (end 111 49.9) (width 0.2) (layer "F.Cu") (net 36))
 (segment (start 98.6 64.8) (end 105.9 64.8) (width 0.2) (layer "F.Cu") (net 36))
 (segment (start 105.9 64.8) (end 106 64.7) (width 0.2) (layer "F.Cu") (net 36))
 (segment (start 111 49.9) (end 117.9 49.9) (width 0.2) (layer "F.Cu") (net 36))
 (segment (start 117.9 49.9) (end 120.5 52.5) (width 0.2) (layer "F.Cu") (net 36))
 (segment (start 98.415 64.95) (end 98.4 65) (width 0.2) (layer "F.Cu") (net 36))
 (segment (start 106 64.7) (end 106 54.9) (width 0.2) (layer "F.Cu") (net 36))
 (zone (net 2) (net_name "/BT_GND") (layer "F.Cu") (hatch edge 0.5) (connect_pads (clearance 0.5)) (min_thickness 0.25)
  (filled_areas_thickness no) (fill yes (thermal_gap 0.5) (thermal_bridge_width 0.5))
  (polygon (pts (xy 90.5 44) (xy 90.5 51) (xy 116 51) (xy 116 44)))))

